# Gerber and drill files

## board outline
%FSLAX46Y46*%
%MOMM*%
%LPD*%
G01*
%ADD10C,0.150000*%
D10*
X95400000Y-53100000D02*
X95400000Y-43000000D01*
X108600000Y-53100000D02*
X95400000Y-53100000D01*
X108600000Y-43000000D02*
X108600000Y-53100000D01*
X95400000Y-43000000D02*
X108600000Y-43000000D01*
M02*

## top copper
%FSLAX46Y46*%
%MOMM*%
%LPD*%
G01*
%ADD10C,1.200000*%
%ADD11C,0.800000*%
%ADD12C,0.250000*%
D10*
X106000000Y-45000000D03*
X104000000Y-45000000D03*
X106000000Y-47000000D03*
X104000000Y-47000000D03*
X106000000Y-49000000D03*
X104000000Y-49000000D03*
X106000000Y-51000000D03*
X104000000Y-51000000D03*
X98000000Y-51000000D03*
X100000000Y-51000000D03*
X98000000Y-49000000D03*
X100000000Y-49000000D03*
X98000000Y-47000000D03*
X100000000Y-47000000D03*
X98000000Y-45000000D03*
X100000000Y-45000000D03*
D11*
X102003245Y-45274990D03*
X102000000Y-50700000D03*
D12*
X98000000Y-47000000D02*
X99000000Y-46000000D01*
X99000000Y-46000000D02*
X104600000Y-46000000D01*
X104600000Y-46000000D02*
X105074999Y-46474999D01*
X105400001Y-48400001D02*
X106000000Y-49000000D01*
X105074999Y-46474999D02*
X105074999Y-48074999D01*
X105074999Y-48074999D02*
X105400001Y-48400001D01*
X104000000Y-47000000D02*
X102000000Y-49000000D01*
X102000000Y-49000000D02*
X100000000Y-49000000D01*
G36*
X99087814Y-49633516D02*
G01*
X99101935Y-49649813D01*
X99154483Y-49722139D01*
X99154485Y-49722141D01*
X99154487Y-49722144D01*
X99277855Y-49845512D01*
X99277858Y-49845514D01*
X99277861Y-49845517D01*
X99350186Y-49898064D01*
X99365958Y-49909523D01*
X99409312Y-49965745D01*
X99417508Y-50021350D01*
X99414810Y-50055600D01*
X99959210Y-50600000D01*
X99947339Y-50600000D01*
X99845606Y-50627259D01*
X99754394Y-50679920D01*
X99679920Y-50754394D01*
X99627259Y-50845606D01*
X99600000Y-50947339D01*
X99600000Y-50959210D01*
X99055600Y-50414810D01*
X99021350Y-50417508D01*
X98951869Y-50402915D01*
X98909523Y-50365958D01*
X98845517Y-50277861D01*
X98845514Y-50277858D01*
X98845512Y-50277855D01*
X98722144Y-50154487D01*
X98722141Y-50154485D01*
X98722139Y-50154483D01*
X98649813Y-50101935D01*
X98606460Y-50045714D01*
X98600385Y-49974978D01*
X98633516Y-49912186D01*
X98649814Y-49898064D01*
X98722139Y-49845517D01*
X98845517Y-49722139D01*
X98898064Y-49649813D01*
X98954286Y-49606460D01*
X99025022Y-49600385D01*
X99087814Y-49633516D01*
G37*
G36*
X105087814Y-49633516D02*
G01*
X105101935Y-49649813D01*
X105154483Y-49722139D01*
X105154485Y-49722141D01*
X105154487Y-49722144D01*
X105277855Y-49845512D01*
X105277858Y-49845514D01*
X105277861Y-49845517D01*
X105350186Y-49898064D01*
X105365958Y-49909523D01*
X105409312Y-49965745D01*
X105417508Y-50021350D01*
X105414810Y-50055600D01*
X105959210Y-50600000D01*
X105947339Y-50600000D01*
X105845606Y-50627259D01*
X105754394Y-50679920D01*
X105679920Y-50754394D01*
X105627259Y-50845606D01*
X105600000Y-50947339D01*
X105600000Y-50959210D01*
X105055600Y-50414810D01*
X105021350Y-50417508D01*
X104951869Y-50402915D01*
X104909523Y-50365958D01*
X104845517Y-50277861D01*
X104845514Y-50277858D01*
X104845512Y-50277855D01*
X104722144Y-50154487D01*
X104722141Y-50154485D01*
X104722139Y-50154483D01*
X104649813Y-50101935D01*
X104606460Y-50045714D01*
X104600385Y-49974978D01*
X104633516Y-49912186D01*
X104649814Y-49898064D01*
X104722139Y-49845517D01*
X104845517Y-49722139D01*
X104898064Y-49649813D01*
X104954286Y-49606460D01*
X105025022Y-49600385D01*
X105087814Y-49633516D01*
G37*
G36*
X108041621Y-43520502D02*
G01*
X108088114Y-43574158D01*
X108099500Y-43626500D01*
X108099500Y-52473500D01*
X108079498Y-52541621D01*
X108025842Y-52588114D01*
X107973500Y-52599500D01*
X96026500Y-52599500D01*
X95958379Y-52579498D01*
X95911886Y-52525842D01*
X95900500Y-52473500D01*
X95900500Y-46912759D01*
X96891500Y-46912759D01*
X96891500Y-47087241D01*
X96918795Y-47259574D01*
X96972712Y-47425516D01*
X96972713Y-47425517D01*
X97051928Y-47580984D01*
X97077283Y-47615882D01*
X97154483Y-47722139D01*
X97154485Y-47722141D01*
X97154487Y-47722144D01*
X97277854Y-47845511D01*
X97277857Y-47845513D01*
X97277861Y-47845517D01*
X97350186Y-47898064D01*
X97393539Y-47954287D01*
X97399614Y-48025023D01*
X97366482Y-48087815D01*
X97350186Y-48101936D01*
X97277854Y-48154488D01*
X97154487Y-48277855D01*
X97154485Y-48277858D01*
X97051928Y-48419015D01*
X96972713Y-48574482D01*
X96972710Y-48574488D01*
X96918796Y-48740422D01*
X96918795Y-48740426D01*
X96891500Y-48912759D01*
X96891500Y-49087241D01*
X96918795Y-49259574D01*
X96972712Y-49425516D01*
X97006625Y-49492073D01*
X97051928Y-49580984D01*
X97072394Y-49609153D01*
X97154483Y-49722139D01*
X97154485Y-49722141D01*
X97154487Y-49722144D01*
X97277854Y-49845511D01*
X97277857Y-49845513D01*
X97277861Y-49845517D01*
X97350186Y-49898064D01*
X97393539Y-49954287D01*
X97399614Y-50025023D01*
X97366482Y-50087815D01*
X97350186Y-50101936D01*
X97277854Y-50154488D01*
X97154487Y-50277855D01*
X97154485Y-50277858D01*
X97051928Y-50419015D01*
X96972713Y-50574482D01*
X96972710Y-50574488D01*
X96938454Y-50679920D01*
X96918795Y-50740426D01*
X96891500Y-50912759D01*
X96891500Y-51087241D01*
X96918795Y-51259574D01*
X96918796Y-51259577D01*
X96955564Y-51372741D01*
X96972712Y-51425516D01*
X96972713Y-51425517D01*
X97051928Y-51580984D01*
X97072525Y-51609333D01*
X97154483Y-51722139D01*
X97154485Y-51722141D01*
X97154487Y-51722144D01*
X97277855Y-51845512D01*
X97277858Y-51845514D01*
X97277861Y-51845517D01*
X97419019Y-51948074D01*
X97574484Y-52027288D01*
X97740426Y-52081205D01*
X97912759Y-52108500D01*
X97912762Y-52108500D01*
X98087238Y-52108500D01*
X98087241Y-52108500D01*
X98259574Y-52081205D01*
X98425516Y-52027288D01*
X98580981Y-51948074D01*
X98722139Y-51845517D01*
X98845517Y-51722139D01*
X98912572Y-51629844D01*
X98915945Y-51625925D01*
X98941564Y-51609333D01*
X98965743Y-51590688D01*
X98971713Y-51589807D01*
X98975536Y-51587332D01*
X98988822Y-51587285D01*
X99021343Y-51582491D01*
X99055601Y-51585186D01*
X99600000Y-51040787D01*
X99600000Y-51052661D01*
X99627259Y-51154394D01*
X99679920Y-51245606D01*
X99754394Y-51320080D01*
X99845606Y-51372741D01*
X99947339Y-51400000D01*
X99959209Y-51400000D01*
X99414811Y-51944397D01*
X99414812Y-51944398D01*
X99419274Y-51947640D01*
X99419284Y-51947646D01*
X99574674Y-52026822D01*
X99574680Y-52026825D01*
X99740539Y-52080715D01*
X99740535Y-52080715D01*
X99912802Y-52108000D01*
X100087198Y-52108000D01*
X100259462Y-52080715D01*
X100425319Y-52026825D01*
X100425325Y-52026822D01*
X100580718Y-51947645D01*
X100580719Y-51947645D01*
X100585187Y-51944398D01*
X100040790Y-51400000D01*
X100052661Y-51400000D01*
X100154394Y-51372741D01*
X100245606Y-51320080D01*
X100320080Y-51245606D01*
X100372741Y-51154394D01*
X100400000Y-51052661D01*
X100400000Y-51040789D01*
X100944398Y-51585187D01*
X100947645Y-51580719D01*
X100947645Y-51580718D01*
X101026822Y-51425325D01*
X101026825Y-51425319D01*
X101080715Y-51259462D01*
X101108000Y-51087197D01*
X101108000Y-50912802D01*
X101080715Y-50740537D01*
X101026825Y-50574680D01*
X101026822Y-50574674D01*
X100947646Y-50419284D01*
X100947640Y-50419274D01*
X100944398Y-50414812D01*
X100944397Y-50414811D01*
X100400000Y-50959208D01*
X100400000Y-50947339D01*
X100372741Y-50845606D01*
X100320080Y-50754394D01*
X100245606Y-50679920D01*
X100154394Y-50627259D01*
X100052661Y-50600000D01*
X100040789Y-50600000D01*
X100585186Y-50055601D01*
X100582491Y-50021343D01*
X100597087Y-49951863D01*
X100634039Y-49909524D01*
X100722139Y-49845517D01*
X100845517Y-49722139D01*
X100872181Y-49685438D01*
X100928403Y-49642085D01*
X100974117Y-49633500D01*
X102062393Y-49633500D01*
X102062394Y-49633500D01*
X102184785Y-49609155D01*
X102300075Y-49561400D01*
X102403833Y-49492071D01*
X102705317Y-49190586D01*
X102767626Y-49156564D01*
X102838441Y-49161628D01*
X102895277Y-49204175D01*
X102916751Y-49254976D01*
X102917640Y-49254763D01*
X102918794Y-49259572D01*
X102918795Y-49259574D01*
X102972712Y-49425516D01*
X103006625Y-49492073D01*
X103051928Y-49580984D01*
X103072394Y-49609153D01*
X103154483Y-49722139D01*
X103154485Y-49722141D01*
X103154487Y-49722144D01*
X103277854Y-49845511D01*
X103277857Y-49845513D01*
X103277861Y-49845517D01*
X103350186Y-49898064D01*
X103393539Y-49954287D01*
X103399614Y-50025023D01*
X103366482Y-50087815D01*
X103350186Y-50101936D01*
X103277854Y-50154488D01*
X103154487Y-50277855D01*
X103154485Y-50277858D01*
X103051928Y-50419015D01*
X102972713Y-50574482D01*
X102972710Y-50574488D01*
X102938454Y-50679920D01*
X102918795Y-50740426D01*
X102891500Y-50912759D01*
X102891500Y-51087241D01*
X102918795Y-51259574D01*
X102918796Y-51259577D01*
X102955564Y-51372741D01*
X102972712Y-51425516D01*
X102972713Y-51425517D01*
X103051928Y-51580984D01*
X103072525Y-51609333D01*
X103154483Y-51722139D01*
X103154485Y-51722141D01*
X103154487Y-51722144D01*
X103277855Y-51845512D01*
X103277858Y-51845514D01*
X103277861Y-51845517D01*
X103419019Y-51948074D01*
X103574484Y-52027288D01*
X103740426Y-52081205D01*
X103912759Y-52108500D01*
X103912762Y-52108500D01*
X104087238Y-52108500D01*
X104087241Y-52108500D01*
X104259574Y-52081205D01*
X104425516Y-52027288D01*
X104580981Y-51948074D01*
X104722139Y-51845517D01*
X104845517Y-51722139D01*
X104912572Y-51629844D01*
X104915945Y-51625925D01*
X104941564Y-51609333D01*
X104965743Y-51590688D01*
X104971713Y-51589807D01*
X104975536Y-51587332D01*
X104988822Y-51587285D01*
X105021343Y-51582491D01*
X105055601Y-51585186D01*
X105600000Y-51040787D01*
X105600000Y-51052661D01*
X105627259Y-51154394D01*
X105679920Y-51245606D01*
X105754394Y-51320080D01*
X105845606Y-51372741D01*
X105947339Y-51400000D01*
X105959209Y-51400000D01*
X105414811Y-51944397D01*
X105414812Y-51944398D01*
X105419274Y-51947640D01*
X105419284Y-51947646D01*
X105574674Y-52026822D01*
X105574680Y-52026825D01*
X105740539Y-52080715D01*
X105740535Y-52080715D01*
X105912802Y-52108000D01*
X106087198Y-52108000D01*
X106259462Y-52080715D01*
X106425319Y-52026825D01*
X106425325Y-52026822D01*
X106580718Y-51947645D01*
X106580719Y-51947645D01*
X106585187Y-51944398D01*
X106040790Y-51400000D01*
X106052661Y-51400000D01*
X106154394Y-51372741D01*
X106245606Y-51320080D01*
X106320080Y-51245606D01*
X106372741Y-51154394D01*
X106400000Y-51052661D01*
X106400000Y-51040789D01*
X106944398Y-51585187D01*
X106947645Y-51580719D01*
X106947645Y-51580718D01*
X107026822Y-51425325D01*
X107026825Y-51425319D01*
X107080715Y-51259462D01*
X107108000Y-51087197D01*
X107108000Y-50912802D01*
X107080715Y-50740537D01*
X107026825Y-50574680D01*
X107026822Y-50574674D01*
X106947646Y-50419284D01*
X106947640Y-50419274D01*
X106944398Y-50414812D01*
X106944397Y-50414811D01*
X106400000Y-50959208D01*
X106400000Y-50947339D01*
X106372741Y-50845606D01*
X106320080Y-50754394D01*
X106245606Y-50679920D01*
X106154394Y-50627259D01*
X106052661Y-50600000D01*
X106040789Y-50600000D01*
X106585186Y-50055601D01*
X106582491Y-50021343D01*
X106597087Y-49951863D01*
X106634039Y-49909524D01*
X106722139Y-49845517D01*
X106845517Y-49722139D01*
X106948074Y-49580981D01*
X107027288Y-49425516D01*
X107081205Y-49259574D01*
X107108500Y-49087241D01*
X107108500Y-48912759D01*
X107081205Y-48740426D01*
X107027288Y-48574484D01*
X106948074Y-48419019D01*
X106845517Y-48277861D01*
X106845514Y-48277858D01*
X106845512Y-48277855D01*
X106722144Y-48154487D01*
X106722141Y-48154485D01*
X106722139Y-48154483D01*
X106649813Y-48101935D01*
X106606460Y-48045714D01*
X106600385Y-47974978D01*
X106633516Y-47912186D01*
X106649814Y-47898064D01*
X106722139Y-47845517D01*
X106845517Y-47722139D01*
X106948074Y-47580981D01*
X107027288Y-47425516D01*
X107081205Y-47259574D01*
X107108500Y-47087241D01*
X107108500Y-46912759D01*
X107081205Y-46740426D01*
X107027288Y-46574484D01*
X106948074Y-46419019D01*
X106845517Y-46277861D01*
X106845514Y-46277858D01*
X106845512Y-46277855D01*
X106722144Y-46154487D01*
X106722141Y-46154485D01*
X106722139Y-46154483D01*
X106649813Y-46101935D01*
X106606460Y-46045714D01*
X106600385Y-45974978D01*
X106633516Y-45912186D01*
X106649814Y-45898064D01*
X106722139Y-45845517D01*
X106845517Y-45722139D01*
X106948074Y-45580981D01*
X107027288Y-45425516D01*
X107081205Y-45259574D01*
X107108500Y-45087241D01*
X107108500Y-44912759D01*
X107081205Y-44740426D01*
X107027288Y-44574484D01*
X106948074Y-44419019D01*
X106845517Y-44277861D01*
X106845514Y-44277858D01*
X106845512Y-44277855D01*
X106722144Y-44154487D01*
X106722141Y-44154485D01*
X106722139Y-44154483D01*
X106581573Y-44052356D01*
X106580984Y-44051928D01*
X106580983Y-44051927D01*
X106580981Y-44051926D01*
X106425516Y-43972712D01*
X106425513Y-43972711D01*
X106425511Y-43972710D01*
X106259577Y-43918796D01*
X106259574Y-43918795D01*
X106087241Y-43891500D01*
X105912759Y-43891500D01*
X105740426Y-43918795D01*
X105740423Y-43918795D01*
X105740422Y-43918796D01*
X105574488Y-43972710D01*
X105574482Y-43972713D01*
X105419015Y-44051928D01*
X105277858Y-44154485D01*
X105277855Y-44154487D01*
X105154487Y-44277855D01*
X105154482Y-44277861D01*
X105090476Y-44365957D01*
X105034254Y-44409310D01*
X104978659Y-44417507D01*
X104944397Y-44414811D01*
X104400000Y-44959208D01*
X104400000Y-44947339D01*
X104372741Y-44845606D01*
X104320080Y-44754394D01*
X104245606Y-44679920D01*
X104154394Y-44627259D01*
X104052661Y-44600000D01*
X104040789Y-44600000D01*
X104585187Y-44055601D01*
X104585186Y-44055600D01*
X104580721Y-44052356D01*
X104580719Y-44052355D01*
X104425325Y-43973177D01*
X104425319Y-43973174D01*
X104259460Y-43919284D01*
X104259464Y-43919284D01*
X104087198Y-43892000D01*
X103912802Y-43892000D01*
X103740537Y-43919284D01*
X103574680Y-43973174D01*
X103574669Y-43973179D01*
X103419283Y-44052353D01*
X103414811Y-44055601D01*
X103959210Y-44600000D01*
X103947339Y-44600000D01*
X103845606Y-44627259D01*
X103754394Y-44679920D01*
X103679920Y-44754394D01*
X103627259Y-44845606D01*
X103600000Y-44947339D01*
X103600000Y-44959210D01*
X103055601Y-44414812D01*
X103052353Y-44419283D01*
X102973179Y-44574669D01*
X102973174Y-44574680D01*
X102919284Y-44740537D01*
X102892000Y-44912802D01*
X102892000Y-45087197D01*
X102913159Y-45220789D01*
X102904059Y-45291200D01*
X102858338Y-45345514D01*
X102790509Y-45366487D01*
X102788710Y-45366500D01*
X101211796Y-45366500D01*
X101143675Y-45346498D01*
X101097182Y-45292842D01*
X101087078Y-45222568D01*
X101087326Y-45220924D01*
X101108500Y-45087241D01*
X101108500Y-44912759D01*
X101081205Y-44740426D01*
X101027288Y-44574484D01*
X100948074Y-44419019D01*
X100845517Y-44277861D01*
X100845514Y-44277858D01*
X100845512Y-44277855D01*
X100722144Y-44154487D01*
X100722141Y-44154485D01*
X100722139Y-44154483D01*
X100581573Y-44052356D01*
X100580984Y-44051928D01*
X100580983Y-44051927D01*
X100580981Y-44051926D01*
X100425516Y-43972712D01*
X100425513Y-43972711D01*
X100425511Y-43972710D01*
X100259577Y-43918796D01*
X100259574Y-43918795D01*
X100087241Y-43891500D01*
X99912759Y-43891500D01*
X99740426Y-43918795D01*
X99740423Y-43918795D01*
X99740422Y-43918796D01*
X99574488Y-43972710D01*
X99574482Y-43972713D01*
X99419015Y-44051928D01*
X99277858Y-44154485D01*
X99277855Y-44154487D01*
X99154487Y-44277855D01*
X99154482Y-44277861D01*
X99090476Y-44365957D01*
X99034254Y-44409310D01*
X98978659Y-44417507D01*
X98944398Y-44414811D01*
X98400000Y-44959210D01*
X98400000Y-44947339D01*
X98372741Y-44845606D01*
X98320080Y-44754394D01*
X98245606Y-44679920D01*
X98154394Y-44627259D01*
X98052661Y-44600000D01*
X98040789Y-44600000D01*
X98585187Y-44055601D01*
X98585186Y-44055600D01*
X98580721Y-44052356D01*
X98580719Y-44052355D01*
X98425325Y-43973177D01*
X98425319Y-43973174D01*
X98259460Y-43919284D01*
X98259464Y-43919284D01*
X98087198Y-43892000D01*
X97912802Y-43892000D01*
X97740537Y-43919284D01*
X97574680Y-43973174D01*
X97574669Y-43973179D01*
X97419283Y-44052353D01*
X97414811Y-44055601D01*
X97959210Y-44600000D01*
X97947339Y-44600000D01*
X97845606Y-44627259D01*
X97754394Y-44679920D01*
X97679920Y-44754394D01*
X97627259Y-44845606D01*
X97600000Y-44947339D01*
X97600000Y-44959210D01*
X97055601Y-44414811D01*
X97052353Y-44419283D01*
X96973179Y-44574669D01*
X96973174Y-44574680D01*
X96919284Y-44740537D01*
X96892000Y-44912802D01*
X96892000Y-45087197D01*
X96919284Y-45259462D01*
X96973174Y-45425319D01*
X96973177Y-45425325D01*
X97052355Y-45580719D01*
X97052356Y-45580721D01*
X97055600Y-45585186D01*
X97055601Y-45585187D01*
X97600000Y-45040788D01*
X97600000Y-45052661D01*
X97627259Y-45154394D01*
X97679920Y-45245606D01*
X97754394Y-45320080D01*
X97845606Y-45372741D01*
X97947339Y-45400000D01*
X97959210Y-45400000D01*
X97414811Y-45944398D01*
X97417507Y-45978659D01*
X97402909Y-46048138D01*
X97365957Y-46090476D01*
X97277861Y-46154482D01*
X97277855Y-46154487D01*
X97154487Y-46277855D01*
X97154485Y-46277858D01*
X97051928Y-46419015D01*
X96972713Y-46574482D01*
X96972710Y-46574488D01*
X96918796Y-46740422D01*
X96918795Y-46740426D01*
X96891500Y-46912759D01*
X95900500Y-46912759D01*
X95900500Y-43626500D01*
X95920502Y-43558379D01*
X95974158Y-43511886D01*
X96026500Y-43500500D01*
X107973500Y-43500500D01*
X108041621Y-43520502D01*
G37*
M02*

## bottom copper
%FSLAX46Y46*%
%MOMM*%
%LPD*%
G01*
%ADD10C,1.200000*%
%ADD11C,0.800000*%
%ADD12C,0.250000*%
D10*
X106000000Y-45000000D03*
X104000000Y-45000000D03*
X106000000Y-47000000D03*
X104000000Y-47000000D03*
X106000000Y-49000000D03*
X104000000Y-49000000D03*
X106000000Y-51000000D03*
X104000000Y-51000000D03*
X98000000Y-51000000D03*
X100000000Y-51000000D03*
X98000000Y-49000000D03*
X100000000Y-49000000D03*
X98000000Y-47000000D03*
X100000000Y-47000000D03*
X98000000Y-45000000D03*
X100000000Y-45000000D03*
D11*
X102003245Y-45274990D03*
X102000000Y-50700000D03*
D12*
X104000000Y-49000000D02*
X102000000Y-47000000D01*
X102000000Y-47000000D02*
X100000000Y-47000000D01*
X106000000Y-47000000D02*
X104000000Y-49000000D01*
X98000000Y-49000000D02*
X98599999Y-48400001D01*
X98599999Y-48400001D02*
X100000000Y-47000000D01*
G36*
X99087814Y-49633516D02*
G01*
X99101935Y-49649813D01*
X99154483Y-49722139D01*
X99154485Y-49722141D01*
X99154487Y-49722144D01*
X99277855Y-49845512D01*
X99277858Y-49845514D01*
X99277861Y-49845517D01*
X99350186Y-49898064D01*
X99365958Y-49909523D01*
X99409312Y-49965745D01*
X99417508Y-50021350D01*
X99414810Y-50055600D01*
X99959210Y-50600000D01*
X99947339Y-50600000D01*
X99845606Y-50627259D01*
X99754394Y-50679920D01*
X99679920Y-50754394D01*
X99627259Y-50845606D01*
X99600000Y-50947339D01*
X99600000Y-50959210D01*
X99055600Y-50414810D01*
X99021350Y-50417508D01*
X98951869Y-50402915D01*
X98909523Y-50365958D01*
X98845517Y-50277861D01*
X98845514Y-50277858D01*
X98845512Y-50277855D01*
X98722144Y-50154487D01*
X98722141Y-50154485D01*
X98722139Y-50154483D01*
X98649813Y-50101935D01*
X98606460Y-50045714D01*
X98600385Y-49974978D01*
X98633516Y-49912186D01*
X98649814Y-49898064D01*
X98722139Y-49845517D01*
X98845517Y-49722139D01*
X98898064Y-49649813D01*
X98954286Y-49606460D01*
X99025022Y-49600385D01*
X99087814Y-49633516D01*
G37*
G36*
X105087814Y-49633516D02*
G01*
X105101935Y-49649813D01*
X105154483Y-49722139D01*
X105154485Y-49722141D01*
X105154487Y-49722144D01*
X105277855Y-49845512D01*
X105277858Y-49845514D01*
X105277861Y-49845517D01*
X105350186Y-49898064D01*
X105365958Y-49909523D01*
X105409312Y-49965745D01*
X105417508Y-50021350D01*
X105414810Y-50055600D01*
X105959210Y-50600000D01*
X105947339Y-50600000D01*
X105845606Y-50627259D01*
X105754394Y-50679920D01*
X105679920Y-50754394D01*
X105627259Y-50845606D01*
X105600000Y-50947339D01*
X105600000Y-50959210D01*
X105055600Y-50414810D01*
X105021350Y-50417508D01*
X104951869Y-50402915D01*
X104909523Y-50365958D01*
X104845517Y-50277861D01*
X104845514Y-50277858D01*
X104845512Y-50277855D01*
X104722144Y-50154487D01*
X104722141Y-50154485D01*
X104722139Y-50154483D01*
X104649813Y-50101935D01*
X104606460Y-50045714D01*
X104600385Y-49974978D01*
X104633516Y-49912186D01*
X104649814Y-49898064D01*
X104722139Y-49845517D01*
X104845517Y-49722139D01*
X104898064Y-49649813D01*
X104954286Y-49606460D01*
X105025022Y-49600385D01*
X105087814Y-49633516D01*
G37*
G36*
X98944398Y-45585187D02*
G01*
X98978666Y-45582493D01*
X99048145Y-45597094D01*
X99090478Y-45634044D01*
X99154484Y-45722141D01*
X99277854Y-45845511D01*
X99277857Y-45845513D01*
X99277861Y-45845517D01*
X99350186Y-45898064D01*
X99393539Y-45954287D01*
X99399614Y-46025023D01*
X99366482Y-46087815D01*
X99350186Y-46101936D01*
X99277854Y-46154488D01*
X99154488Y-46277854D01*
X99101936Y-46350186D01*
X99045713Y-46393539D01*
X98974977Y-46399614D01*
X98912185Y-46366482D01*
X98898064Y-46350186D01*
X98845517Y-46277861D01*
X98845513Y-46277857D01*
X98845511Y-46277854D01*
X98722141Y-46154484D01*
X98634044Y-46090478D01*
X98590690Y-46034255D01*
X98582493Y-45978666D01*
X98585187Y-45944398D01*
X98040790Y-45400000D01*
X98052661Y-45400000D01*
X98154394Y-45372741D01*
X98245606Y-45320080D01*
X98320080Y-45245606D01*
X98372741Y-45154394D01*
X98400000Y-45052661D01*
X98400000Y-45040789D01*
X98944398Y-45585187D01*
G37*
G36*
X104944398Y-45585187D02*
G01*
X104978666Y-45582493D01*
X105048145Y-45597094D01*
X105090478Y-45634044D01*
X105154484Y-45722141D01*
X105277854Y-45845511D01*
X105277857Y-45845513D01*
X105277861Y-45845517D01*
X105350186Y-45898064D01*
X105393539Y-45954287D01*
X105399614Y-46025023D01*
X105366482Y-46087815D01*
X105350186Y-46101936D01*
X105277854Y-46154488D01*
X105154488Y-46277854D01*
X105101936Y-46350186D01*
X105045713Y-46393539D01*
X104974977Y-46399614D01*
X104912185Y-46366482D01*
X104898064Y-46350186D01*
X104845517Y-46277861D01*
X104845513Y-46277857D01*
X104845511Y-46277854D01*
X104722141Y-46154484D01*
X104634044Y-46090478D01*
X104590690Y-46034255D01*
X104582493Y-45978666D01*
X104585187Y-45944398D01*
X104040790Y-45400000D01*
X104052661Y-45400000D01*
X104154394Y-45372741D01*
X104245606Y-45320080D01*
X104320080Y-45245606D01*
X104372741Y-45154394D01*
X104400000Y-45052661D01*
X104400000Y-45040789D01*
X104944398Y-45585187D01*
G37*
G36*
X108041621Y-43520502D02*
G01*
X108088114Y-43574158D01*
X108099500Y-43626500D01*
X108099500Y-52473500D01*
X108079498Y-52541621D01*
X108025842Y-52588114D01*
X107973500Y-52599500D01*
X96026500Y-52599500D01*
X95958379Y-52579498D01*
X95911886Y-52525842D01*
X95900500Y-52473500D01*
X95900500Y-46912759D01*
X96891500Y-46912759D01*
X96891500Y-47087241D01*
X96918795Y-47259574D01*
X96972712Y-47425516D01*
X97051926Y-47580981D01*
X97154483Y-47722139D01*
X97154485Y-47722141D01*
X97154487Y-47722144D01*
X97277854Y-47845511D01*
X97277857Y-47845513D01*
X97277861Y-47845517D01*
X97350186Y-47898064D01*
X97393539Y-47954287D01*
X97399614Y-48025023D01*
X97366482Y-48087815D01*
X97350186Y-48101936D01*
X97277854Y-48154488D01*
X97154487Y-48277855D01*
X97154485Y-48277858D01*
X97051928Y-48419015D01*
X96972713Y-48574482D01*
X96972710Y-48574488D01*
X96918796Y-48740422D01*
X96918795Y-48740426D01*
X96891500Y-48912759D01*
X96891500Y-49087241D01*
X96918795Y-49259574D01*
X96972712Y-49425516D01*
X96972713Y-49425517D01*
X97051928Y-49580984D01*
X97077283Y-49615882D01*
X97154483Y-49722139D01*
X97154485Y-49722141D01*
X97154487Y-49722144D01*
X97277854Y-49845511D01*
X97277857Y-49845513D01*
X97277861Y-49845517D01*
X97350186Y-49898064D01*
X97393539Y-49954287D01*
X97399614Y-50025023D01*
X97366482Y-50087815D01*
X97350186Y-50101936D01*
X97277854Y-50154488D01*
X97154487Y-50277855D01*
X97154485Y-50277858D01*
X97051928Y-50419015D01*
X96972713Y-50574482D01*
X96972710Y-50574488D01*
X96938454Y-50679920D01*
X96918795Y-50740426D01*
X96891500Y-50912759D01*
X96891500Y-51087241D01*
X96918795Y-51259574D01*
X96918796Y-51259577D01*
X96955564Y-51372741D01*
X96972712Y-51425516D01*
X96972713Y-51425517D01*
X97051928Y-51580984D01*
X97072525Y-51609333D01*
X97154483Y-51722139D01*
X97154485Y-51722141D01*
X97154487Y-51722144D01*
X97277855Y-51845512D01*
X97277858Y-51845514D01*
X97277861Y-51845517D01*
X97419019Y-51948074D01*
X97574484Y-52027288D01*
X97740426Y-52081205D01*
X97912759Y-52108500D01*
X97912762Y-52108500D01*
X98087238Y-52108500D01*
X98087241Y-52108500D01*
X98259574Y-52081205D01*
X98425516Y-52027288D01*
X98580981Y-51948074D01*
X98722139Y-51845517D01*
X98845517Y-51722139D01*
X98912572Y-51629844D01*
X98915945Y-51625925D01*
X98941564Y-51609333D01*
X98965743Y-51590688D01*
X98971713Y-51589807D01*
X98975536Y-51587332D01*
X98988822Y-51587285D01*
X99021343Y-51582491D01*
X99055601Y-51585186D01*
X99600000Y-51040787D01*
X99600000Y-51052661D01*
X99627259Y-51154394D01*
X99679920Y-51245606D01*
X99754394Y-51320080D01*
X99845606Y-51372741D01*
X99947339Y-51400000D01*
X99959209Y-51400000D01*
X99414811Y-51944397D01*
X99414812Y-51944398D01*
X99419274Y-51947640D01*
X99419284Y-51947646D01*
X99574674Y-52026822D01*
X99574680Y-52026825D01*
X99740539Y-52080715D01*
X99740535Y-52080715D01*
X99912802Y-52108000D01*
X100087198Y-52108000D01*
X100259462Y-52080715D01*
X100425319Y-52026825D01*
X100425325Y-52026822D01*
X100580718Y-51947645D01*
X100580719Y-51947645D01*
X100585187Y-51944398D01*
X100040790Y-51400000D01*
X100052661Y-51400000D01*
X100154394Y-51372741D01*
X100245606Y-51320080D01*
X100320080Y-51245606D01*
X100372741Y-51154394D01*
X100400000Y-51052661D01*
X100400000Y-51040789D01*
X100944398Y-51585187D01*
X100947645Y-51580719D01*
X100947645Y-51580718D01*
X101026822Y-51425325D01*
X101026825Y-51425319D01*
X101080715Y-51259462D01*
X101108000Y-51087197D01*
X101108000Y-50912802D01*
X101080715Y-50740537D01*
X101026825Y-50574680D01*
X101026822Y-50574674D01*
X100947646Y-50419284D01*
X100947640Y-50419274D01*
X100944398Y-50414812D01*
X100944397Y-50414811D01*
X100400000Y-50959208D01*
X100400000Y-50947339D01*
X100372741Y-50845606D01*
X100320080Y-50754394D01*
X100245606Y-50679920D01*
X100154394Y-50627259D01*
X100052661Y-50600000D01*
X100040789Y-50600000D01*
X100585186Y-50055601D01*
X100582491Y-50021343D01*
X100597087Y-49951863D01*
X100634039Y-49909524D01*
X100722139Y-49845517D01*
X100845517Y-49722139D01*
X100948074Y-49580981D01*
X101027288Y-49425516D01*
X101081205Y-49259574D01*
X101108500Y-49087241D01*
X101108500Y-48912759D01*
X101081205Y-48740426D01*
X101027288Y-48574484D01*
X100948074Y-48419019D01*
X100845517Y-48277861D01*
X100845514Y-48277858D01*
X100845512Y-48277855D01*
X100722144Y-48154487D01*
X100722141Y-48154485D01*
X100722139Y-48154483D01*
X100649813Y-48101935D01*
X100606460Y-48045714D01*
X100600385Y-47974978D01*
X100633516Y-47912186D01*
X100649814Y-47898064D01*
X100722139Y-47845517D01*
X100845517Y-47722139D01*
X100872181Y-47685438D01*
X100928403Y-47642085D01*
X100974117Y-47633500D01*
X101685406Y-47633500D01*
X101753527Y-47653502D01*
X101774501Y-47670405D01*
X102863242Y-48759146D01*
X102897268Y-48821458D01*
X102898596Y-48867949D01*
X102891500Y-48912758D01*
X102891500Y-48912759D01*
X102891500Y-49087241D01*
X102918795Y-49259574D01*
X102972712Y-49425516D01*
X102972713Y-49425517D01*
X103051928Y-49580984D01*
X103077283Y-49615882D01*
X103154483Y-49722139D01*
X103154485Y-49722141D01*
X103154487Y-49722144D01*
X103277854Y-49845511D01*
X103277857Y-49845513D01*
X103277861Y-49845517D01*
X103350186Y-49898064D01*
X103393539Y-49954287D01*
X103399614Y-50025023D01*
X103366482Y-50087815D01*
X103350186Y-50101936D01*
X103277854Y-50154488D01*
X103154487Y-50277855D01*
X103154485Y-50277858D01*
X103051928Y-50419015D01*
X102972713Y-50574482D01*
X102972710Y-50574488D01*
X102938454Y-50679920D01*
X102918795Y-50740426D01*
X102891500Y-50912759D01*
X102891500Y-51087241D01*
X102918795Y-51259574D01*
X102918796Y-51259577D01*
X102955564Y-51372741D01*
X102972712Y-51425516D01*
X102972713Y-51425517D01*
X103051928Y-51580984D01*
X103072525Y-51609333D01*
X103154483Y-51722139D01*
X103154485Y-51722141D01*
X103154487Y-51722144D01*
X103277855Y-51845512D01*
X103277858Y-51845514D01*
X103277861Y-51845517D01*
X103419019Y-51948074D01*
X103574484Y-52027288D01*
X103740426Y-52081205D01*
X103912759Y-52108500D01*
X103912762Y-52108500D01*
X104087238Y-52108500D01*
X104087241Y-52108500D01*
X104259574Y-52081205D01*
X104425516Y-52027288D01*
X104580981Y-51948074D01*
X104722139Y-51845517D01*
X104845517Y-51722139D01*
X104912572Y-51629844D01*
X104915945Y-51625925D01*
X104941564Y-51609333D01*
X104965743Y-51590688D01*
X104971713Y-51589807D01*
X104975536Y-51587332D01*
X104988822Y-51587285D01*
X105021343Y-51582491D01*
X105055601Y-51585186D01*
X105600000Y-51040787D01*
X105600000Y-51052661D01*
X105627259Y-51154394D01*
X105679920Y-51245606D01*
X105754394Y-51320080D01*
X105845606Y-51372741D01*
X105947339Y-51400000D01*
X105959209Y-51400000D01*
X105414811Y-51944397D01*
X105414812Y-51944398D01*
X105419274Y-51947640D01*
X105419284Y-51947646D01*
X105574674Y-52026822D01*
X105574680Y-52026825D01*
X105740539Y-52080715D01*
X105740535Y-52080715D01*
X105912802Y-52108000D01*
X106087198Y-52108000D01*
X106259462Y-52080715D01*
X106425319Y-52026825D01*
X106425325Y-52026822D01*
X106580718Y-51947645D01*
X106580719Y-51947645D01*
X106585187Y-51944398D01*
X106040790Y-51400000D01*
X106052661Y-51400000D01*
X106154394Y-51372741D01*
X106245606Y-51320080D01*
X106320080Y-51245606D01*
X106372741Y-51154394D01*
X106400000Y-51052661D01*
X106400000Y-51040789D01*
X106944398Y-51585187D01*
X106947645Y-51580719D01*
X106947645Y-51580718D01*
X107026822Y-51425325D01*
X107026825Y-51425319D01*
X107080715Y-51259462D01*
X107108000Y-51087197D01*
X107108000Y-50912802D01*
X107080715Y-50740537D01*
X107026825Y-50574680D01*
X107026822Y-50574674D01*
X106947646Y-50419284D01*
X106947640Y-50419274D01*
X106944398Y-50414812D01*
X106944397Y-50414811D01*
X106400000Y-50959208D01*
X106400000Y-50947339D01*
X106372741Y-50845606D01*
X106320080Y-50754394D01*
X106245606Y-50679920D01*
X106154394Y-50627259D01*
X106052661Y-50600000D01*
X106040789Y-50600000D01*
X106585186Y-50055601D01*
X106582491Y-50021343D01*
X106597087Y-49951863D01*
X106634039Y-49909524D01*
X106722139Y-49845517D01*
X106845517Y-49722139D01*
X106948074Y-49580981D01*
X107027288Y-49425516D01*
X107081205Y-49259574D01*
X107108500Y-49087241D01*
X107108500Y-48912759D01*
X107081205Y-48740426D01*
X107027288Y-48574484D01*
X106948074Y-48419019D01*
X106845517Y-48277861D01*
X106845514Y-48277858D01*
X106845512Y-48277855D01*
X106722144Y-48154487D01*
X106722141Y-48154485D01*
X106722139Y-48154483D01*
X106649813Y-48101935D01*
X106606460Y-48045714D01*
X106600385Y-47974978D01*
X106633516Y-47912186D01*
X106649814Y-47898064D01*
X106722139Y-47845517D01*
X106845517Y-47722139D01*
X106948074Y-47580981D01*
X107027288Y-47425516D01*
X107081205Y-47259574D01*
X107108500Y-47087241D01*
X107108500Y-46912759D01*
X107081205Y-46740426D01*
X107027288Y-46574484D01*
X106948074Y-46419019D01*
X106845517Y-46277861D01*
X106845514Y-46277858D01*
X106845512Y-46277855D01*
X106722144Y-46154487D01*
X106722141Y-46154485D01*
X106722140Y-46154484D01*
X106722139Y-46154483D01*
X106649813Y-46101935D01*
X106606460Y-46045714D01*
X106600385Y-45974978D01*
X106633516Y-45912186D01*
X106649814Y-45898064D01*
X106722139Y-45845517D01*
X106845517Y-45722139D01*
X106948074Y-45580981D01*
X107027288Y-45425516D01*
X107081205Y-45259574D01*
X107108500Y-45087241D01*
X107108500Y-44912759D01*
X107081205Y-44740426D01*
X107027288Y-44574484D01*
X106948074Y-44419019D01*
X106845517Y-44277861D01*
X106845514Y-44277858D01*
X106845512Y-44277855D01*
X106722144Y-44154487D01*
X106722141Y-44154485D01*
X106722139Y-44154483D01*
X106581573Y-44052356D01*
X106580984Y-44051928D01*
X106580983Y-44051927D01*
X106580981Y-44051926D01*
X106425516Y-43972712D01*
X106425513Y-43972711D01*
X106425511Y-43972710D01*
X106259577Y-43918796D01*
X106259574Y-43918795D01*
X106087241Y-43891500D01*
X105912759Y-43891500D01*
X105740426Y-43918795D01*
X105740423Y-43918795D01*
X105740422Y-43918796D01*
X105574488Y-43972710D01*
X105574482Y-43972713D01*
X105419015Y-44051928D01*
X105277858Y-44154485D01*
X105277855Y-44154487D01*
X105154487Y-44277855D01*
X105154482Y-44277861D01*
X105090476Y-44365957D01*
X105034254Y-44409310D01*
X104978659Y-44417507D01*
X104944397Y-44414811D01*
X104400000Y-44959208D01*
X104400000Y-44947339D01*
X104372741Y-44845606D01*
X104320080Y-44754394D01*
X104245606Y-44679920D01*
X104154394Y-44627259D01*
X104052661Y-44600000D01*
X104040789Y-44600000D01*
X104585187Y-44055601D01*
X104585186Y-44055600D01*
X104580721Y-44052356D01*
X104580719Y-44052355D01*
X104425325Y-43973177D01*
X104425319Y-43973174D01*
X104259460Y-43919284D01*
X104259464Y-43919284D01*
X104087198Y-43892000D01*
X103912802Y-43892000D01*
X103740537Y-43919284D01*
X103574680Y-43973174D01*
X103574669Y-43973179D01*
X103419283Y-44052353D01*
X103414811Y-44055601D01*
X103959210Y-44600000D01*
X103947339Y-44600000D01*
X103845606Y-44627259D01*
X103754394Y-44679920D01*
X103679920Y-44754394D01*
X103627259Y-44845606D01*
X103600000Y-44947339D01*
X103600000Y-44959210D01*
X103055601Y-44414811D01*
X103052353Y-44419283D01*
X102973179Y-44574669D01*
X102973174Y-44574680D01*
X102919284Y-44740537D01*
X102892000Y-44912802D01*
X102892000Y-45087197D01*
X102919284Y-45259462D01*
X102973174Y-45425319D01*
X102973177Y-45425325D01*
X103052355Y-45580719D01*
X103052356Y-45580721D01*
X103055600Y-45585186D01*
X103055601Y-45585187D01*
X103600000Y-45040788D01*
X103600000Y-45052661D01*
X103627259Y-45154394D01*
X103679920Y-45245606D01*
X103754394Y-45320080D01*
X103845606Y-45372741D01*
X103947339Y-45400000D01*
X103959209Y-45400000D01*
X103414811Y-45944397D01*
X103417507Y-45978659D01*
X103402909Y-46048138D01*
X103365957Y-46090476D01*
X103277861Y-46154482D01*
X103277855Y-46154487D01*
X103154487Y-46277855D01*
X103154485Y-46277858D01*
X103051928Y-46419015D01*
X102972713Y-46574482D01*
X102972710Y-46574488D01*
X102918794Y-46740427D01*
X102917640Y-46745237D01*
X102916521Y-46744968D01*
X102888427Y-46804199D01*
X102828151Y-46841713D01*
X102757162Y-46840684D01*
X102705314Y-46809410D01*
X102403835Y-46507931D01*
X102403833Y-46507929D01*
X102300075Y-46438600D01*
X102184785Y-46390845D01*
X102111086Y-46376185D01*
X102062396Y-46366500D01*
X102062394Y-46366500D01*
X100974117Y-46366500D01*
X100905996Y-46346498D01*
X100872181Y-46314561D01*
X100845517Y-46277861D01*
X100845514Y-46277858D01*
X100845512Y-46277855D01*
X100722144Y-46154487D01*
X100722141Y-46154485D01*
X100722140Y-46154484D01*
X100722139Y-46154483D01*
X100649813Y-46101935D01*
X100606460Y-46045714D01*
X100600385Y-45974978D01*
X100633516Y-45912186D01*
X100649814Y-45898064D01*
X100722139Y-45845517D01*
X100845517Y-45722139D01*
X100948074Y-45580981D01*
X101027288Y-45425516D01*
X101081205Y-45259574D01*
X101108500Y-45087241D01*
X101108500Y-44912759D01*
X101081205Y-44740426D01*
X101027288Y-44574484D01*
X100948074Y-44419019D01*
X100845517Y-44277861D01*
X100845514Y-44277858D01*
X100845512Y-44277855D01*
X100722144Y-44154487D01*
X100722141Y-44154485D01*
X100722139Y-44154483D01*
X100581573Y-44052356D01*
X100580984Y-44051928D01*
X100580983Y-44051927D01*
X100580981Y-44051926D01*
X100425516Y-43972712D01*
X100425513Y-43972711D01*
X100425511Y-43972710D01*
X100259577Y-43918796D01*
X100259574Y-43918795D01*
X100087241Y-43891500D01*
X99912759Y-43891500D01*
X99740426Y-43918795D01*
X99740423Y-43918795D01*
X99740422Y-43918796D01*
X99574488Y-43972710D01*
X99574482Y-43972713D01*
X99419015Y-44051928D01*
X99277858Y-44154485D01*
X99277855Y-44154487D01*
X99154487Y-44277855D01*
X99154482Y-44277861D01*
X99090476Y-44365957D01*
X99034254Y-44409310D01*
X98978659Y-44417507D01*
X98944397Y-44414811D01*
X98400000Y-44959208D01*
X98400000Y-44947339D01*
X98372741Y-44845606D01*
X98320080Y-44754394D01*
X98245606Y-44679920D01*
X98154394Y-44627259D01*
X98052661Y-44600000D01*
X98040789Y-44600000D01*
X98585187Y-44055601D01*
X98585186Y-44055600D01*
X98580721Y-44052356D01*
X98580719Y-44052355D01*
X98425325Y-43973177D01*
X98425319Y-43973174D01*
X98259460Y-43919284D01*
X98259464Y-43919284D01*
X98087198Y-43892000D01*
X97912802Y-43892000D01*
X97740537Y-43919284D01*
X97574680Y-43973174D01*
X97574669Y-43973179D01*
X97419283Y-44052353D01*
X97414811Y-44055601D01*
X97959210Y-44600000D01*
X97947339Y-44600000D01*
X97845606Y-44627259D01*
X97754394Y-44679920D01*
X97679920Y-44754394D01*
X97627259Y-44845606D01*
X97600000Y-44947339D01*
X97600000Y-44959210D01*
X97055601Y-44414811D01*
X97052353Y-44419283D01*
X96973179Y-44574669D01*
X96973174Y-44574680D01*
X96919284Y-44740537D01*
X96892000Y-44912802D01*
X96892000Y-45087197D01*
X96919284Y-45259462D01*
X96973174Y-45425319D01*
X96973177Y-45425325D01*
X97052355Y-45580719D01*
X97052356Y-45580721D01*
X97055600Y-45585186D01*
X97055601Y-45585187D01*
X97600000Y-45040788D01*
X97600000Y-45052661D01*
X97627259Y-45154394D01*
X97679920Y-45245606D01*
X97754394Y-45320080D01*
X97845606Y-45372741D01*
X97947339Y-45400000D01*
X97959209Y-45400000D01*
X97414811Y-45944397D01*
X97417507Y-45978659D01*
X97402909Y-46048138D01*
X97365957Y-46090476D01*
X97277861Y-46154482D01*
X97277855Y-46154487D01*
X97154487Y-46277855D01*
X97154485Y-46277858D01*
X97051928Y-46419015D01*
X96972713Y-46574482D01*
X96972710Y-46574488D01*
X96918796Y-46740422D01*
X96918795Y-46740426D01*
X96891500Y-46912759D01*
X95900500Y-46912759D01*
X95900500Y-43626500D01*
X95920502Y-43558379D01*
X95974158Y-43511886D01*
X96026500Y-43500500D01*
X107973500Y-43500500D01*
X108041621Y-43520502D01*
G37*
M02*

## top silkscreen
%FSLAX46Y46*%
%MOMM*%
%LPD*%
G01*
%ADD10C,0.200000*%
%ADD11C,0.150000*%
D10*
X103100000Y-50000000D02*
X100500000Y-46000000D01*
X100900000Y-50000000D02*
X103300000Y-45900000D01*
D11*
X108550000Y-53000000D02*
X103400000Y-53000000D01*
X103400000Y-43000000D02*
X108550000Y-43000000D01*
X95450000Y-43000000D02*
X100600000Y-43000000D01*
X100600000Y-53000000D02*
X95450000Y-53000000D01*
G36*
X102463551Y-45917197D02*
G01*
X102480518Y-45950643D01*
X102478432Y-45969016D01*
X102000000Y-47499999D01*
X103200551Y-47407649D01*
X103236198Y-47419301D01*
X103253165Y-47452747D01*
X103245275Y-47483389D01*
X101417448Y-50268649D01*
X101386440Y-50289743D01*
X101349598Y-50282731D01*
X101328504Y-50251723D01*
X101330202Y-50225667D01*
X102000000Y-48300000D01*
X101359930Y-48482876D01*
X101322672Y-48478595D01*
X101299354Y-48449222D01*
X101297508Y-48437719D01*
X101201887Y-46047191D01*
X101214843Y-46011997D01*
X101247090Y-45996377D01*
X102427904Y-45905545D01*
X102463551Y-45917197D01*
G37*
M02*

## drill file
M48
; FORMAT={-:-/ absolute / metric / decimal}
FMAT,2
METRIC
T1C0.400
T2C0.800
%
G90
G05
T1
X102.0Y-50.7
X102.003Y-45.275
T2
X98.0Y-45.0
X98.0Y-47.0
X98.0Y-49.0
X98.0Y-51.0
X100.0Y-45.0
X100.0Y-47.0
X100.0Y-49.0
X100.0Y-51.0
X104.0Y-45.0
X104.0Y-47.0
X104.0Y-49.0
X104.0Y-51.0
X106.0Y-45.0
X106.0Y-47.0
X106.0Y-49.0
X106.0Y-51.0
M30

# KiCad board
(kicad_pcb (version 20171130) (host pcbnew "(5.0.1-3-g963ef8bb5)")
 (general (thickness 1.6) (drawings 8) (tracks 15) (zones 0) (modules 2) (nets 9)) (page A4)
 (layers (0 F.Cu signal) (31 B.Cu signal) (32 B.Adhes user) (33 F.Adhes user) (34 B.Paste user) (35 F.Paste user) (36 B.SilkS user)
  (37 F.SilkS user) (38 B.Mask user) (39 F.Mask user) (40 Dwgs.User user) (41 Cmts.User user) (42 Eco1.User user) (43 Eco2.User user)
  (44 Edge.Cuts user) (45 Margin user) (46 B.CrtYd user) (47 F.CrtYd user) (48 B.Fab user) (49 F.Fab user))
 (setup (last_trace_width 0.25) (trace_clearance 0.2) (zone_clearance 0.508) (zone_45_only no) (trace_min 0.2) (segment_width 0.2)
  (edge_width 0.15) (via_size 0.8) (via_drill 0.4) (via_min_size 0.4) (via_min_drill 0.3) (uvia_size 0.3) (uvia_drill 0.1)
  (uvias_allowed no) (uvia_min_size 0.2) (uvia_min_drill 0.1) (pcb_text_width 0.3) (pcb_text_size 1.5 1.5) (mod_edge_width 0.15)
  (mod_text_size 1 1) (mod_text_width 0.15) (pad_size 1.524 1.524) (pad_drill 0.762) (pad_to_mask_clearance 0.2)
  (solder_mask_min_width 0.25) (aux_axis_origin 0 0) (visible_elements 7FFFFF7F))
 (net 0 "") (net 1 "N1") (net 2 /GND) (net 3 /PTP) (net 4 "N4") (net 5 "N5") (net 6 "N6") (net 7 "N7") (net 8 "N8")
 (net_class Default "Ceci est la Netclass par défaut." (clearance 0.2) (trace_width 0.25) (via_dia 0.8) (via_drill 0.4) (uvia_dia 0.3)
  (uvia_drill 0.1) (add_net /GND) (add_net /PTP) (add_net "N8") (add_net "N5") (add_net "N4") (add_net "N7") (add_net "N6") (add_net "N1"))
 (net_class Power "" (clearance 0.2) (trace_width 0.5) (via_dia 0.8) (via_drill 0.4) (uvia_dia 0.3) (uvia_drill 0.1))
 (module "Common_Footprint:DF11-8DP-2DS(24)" (layer F.Cu) (at 105 48 270)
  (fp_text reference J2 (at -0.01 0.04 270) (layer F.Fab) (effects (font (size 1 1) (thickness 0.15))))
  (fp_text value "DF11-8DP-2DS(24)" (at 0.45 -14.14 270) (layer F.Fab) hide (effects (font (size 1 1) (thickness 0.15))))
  (fp_line (start 5 -3.55) (end 5 1.6) (layer F.SilkS) (width 0.15))
  (fp_line (start -5 1.6) (end -5 -3.55) (layer F.SilkS) (width 0.15))
  (pad 8 thru_hole circle (at -3 -1 270) (size 1.2 1.2) (drill 0.8) (layers *.Cu *.Mask) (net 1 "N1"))
  (pad 7 thru_hole circle (at -3 1 270) (size 1.2 1.2) (drill 0.8) (layers *.Cu *.Mask) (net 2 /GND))
  (pad 6 thru_hole circle (at -1 -1 270) (size 1.2 1.2) (drill 0.8) (layers *.Cu *.Mask) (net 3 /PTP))
  (pad 5 thru_hole circle (at -1 1 270) (size 1.2 1.2) (drill 0.8) (layers *.Cu *.Mask) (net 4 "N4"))
  (pad 4 thru_hole circle (at 1 -1 270) (size 1.2 1.2) (drill 0.8) (layers *.Cu *.Mask) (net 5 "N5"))
  (pad 3 thru_hole circle (at 1 1 270) (size 1.2 1.2) (drill 0.8) (layers *.Cu *.Mask) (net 3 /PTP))
  (pad 2 thru_hole circle (at 3 -1 270) (size 1.2 1.2) (drill 0.8) (layers *.Cu *.Mask) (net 2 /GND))
  (pad 1 thru_hole circle (at 3 1 270) (size 1.2 1.2) (drill 0.8) (layers *.Cu *.Mask) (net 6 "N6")))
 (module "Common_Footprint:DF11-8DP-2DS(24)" (layer F.Cu) (at 99 48 90)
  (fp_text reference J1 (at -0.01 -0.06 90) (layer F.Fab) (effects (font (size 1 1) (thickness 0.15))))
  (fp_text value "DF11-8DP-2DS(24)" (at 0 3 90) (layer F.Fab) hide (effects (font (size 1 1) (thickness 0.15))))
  (fp_line (start 5 -3.55) (end 5 1.6) (layer F.SilkS) (width 0.15))
  (fp_line (start -5 1.6) (end -5 -3.55) (layer F.SilkS) (width 0.15))
  (pad 8 thru_hole circle (at -3 -1 90) (size 1.2 1.2) (drill 0.8) (layers *.Cu *.Mask) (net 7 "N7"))
  (pad 7 thru_hole circle (at -3 1 90) (size 1.2 1.2) (drill 0.8) (layers *.Cu *.Mask) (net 2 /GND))
  (pad 6 thru_hole circle (at -1 -1 90) (size 1.2 1.2) (drill 0.8) (layers *.Cu *.Mask) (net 3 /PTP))
  (pad 5 thru_hole circle (at -1 1 90) (size 1.2 1.2) (drill 0.8) (layers *.Cu *.Mask) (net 4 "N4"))
  (pad 4 thru_hole circle (at 1 -1 90) (size 1.2 1.2) (drill 0.8) (layers *.Cu *.Mask) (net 5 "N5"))
  (pad 3 thru_hole circle (at 1 1 90) (size 1.2 1.2) (drill 0.8) (layers *.Cu *.Mask) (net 3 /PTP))
  (pad 2 thru_hole circle (at 3 -1 90) (size 1.2 1.2) (drill 0.8) (layers *.Cu *.Mask) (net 2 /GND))
  (pad 1 thru_hole circle (at 3 1 90) (size 1.2 1.2) (drill 0.8) (layers *.Cu *.Mask) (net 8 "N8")))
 (gr_line (start 103.1 50) (end 100.5 46) (layer F.SilkS) (width 0.2))
 (gr_line (start 100.9 50) (end 103.3 45.9) (layer F.SilkS) (width 0.2))
 (gr_line (start 95.4 53.1) (end 95.4 43) (layer Edge.Cuts) (width 0.15))
 (gr_line (start 108.6 53.1) (end 95.4 53.1) (layer Edge.Cuts) (width 0.15))
 (gr_line (start 108.6 43) (end 108.6 53.1) (layer Edge.Cuts) (width 0.15))
 (gr_line (start 95.4 43) (end 108.6 43) (layer Edge.Cuts) (width 0.15))
 (segment (start 98 47) (end 99 46) (width 0.25) (layer F.Cu) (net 5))
 (segment (start 99 46) (end 104.6 46) (width 0.25) (layer F.Cu) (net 5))
 (segment (start 104.6 46) (end 105.074999 46.474999) (width 0.25) (layer F.Cu) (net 5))
 (segment (start 105.400001 48.400001) (end 106 49) (width 0.25) (layer F.Cu) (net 5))
 (segment (start 105.074999 46.474999) (end 105.074999 48.074999) (width 0.25) (layer F.Cu) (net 5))
 (segment (start 105.074999 48.074999) (end 105.400001 48.400001) (width 0.25) (layer F.Cu) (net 5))
 (segment (start 104 47) (end 102 49) (width 0.25) (layer F.Cu) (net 4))
 (segment (start 102 49) (end 100 49) (width 0.25) (layer F.Cu) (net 4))
 (via (at 102.003245 45.27499) (size 0.8) (drill 0.4) (layers F.Cu B.Cu) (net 2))
 (via (at 102 50.7) (size 0.8) (drill 0.4) (layers F.Cu B.Cu) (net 2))
 (segment (start 104 49) (end 102 47) (width 0.25) (layer B.Cu) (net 3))
 (segment (start 102 47) (end 100 47) (width 0.25) (layer B.Cu) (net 3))
 (segment (start 106 47) (end 104 49) (width 0.25) (layer B.Cu) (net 3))
 (segment (start 98 49) (end 98.599999 48.400001) (width 0.25) (layer B.Cu) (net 3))
 (segment (start 98.599999 48.400001) (end 100 47) (width 0.25) (layer B.Cu) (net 3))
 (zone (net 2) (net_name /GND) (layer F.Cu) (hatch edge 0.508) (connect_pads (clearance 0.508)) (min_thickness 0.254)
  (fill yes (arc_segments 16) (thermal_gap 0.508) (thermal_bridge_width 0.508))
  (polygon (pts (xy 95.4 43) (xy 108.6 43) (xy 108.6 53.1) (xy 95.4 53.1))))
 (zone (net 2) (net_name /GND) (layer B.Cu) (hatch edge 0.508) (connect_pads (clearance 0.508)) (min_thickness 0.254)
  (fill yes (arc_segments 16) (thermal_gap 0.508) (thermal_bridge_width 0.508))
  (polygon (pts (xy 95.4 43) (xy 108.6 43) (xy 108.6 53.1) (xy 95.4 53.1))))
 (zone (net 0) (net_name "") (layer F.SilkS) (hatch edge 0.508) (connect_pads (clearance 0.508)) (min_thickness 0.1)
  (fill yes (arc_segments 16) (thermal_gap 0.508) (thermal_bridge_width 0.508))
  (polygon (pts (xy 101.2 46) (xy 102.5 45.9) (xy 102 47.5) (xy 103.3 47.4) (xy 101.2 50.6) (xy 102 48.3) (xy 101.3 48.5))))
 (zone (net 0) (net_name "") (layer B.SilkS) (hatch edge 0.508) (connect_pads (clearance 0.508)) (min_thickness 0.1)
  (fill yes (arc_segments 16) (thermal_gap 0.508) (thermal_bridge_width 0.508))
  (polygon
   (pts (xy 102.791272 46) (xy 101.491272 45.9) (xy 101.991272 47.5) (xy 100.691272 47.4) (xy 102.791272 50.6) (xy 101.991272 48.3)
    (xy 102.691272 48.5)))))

